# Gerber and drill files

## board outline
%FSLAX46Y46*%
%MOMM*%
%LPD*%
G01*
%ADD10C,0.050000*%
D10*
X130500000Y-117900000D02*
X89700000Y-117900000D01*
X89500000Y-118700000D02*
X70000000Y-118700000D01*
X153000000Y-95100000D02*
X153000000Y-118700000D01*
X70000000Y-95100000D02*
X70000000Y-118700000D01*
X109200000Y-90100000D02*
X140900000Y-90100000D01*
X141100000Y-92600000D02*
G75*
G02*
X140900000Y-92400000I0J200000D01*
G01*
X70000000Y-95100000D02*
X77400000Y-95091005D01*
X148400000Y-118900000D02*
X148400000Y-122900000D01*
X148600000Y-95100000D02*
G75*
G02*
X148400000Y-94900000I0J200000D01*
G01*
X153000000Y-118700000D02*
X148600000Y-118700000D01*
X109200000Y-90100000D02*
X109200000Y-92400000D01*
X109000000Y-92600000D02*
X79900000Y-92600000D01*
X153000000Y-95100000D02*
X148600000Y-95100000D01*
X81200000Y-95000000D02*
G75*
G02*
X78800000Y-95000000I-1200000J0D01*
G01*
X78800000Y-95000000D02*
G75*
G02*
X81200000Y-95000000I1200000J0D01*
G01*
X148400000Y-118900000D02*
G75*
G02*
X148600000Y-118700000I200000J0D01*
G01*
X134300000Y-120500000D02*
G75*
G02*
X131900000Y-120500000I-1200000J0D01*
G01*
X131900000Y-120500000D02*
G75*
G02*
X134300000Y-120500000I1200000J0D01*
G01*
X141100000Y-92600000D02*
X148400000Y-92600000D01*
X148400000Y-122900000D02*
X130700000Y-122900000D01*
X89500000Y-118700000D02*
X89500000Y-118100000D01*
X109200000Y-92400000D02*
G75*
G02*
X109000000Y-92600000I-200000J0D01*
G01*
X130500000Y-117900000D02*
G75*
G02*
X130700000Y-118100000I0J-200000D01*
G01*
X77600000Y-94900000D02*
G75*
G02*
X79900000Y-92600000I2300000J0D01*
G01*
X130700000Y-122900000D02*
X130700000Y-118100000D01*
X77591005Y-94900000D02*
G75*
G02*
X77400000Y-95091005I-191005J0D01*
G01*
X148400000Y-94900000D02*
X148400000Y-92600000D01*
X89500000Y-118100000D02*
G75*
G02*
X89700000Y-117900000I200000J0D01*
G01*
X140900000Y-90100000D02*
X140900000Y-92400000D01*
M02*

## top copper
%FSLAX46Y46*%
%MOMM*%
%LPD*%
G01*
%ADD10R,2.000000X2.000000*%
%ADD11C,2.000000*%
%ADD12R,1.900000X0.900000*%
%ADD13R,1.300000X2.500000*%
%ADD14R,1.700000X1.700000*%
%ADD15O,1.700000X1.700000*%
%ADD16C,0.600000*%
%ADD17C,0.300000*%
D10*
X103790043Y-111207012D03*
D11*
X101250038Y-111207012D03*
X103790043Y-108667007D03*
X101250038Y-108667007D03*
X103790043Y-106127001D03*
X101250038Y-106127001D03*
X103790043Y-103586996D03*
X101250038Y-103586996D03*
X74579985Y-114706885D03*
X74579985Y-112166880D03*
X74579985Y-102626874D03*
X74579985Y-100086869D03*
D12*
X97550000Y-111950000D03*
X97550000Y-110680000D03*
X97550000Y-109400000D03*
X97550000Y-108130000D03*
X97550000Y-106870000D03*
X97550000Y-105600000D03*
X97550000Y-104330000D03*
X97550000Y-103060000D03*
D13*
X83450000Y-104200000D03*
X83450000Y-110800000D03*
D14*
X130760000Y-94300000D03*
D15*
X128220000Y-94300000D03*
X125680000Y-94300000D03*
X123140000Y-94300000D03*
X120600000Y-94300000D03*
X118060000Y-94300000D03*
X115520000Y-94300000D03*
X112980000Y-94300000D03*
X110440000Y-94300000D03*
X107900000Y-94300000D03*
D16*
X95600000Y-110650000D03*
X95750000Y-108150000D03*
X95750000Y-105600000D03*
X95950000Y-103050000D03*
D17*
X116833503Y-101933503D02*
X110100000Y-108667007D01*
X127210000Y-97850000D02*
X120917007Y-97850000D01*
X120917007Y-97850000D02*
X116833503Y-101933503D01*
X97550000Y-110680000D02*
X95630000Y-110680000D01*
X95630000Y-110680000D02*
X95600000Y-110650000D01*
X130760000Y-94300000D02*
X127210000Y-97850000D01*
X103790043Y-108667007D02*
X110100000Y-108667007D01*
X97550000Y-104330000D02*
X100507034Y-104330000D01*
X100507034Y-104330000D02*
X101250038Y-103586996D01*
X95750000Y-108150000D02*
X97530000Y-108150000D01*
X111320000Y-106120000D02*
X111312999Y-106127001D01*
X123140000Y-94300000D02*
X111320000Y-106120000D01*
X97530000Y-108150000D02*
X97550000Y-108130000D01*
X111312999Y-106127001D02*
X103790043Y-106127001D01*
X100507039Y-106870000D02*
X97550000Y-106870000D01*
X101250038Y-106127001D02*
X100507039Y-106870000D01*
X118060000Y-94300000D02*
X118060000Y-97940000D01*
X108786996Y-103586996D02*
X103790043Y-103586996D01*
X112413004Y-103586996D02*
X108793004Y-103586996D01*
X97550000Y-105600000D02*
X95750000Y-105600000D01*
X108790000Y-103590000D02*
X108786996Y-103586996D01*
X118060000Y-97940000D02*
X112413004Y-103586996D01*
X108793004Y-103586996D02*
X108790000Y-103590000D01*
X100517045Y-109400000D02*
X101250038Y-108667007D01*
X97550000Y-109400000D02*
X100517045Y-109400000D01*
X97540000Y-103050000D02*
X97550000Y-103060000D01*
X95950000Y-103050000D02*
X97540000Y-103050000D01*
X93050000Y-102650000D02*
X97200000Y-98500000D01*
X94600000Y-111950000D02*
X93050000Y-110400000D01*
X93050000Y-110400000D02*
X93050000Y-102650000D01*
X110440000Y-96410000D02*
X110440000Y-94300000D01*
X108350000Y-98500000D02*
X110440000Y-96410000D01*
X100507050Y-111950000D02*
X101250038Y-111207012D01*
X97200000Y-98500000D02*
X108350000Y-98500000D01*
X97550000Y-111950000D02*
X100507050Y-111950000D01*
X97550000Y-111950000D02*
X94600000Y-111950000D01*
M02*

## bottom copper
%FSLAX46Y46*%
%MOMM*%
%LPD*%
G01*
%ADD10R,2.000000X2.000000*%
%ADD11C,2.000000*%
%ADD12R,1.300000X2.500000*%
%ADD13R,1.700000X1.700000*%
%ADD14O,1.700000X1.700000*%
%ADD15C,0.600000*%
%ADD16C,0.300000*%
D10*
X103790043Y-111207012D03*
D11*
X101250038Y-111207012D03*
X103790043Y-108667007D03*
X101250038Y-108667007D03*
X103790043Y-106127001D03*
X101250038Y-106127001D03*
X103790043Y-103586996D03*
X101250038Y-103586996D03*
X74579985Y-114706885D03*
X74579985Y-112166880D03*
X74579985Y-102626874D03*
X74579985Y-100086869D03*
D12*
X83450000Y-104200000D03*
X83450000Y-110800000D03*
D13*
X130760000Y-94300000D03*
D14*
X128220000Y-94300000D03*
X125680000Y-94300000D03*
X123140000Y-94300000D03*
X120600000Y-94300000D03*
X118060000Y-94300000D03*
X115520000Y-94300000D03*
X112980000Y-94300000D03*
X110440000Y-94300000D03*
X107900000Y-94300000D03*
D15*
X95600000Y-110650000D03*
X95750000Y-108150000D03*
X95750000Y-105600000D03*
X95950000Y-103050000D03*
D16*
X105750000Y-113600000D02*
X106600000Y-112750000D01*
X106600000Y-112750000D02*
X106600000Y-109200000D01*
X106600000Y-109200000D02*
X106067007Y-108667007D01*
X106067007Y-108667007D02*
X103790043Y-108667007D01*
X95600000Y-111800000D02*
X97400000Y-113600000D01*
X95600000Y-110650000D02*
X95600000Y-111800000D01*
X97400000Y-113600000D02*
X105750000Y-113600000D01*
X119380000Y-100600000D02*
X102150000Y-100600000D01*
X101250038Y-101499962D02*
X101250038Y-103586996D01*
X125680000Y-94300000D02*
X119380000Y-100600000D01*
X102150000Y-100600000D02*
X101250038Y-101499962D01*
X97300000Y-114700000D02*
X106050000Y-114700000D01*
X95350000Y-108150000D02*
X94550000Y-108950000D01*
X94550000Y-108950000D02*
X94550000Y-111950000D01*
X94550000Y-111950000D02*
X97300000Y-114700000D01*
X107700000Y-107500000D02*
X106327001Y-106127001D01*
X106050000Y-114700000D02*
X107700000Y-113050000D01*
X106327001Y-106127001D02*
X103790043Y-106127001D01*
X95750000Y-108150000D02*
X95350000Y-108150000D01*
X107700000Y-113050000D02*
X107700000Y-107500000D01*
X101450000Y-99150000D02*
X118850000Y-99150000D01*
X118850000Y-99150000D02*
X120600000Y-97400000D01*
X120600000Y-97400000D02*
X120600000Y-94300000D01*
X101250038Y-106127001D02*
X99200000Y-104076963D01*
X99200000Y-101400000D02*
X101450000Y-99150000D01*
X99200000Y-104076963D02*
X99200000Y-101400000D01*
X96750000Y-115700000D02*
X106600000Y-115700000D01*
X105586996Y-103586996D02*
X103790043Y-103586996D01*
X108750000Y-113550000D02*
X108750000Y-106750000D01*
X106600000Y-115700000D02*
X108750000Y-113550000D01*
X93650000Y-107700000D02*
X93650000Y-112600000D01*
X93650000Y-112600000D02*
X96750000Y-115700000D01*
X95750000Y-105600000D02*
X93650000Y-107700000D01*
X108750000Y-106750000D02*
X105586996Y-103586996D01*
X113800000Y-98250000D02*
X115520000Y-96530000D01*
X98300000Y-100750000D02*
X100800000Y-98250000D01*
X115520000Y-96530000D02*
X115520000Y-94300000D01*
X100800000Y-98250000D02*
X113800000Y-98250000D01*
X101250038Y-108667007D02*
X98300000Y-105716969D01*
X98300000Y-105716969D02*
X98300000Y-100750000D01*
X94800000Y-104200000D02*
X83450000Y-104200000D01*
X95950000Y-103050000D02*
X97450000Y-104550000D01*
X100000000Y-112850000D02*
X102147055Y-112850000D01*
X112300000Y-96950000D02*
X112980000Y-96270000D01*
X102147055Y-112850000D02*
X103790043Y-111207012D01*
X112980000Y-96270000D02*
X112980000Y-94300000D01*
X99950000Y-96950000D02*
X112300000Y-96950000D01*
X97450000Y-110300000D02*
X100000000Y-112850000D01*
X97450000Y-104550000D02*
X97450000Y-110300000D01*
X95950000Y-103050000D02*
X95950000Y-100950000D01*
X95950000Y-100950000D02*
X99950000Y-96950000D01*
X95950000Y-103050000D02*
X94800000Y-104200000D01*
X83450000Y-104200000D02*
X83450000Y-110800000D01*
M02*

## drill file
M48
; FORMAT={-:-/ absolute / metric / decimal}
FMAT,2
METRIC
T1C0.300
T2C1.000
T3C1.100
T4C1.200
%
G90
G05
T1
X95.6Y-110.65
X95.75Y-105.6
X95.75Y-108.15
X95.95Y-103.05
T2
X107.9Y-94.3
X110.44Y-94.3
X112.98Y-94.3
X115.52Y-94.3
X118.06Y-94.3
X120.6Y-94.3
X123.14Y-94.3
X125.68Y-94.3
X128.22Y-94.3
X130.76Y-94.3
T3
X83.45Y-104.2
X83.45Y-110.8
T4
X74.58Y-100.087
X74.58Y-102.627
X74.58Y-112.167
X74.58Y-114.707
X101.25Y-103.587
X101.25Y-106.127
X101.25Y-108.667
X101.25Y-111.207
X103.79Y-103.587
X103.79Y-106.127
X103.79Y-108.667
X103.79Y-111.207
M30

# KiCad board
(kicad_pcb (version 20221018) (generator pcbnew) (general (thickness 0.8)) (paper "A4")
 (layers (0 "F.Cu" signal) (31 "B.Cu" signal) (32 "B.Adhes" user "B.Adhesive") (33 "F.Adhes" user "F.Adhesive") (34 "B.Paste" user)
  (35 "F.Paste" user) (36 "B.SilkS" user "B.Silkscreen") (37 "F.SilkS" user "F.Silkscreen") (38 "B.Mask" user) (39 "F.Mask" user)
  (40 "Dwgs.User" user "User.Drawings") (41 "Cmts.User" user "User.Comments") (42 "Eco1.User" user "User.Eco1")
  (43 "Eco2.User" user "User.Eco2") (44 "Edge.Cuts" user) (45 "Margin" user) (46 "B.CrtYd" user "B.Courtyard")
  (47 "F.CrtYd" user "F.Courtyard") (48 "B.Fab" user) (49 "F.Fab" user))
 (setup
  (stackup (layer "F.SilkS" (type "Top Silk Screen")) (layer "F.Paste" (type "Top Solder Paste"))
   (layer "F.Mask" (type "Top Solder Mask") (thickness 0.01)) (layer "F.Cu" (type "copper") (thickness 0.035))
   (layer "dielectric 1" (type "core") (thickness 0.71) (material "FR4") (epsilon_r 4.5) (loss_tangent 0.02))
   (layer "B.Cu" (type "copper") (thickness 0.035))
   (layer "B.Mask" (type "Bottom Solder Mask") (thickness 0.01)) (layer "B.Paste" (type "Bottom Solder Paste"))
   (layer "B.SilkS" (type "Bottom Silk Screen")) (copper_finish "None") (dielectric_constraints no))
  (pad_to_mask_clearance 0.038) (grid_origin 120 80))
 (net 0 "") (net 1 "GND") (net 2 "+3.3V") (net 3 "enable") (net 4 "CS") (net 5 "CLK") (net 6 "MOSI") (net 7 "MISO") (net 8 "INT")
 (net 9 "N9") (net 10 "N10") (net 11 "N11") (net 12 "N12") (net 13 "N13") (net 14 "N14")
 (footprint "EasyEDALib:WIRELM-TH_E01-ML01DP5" (layer "F.Cu") (at 89.185014 107.396877)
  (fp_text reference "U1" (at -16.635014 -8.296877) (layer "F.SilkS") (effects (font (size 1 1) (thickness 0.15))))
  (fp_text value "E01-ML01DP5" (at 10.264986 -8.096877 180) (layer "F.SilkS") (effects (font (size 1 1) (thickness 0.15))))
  (pad "1" thru_hole rect (at 14.605029 3.810135 180) (size 2 2) (drill 1.2) (layers "*.Cu" "*.Mask") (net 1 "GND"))
  (pad "2" thru_hole circle (at 12.065024 3.810135) (size 2 2) (drill 1.2) (layers "*.Cu" "*.Mask") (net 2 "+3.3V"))
  (pad "3" thru_hole circle (at 14.605029 1.27013) (size 2 2) (drill 1.2) (layers "*.Cu" "*.Mask") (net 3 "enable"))
  (pad "4" thru_hole circle (at 12.065024 1.27013) (size 2 2) (drill 1.2) (layers "*.Cu" "*.Mask") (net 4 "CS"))
  (pad "5" thru_hole circle (at 14.605029 -1.269876) (size 2 2) (drill 1.2) (layers "*.Cu" "*.Mask") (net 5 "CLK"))
  (pad "6" thru_hole circle (at 12.065024 -1.269876) (size 2 2) (drill 1.2) (layers "*.Cu" "*.Mask") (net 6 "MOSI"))
  (pad "7" thru_hole circle (at 14.605029 -3.809881) (size 2 2) (drill 1.2) (layers "*.Cu" "*.Mask") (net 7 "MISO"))
  (pad "8" thru_hole circle (at 12.065024 -3.809881) (size 2 2) (drill 1.2) (layers "*.Cu" "*.Mask") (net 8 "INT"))
  (pad "9" thru_hole circle (at -14.605029 7.310008) (size 2 2) (drill 1.2) (layers "*.Cu" "*.Mask") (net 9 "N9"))
  (pad "10" thru_hole circle (at -14.605029 4.770003) (size 2 2) (drill 1.2) (layers "*.Cu" "*.Mask") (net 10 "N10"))
  (pad "11" thru_hole circle (at -14.605029 -4.770003) (size 2 2) (drill 1.2) (layers "*.Cu" "*.Mask") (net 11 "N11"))
  (pad "12" thru_hole circle (at -14.605029 -7.310008) (size 2 2) (drill 1.2) (layers "*.Cu" "*.Mask") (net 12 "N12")))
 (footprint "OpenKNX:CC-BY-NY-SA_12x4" (layer "F.Cu") (at 141.325111 119.895111)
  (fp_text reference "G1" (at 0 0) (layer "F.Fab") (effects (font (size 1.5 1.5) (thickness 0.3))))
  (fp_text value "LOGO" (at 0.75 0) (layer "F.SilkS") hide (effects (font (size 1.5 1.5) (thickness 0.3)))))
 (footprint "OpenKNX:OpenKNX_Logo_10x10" (layer "F.Cu") (at 139.42 114.81)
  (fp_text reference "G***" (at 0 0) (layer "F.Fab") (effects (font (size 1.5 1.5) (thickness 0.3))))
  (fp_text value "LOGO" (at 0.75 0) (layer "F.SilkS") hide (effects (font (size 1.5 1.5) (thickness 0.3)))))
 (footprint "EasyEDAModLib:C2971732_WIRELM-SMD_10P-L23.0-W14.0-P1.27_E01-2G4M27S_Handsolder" (layer "F.Cu") (at 90.5 107.5 -90)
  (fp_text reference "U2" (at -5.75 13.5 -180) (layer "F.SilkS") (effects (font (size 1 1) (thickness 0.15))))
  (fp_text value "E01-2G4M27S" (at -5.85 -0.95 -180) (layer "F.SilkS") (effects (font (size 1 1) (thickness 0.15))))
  (pad "1" smd rect (at 4.45 -7.05 180) (size 1.9 0.9) (layers "F.Cu" "F.Paste" "F.Mask") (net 2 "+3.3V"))
  (pad "2" smd rect (at 3.18 -7.05 180) (size 1.9 0.9) (layers "F.Cu" "F.Paste" "F.Mask") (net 3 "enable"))
  (pad "3" smd rect (at 1.9 -7.05 180) (size 1.9 0.9) (layers "F.Cu" "F.Paste" "F.Mask") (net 4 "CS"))
  (pad "4" smd rect (at 0.63 -7.05 180) (size 1.9 0.9) (layers "F.Cu" "F.Paste" "F.Mask") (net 5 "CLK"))
  (pad "5" smd rect (at -0.63 -7.05 180) (size 1.9 0.9) (layers "F.Cu" "F.Paste" "F.Mask") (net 6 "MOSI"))
  (pad "6" smd rect (at -1.9 -7.05 180) (size 1.9 0.9) (layers "F.Cu" "F.Paste" "F.Mask") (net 7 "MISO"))
  (pad "7" smd rect (at -3.17 -7.05 180) (size 1.9 0.9) (layers "F.Cu" "F.Paste" "F.Mask") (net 8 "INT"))
  (pad "8" smd rect (at -4.44 -7.05 180) (size 1.9 0.9) (layers "F.Cu" "F.Paste" "F.Mask") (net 1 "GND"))
  (pad "9" thru_hole rect (at -3.3 7.05 180) (size 1.3 2.5) (drill 1.1) (layers "*.Cu" "*.Mask") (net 1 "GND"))
  (pad "10" thru_hole rect (at 3.3 7.05 180) (size 1.3 2.5) (drill 1.1) (layers "*.Cu" "*.Mask") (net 1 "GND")))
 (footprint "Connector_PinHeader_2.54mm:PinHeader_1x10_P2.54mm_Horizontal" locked (layer "B.Cu") (at 130.76 94.3 90)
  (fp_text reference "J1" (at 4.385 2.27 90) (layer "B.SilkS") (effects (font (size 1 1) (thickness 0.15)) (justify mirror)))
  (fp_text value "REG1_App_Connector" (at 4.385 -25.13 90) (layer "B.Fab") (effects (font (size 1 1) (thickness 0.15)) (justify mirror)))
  (pad "1" thru_hole rect locked (at 0 0 90) (size 1.7 1.7) (drill 1) (layers "*.Cu" "*.Mask") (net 3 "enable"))
  (pad "2" thru_hole oval locked (at 0 -2.54 90) (size 1.7 1.7) (drill 1) (layers "*.Cu" "*.Mask") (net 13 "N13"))
  (pad "3" thru_hole oval locked (at 0 -5.08 90) (size 1.7 1.7) (drill 1) (layers "*.Cu" "*.Mask") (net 8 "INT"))
  (pad "4" thru_hole oval locked (at 0 -7.62 90) (size 1.7 1.7) (drill 1) (layers "*.Cu" "*.Mask") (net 5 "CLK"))
  (pad "5" thru_hole oval locked (at 0 -10.16 90) (size 1.7 1.7) (drill 1) (layers "*.Cu" "*.Mask") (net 6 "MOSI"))
  (pad "6" thru_hole oval locked (at 0 -12.7 90) (size 1.7 1.7) (drill 1) (layers "*.Cu" "*.Mask") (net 7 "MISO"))
  (pad "7" thru_hole oval locked (at 0 -15.24 90) (size 1.7 1.7) (drill 1) (layers "*.Cu" "*.Mask") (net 4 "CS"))
  (pad "8" thru_hole oval locked (at 0 -17.78 90) (size 1.7 1.7) (drill 1) (layers "*.Cu" "*.Mask") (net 1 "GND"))
  (pad "9" thru_hole oval locked (at 0 -20.32 90) (size 1.7 1.7) (drill 1) (layers "*.Cu" "*.Mask") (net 2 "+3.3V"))
  (pad "10" thru_hole oval locked (at 0 -22.86 90) (size 1.7 1.7) (drill 1) (layers "*.Cu" "*.Mask") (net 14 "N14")))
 (gr_line (start 130.5 117.9) (end 89.7 117.9) (stroke (width 0.05) (type solid)) (layer "Edge.Cuts"))
 (gr_line (start 89.5 118.7) (end 70 118.7) (stroke (width 0.05) (type solid)) (layer "Edge.Cuts"))
 (gr_line (start 153 95.1) (end 153 118.7) (stroke (width 0.05) (type solid)) (layer "Edge.Cuts"))
 (gr_line (start 70 95.1) (end 70 118.7) (stroke (width 0.05) (type solid)) (layer "Edge.Cuts"))
 (gr_line (start 109.2 90.1) (end 140.9 90.1) (stroke (width 0.05) (type solid)) (layer "Edge.Cuts"))
 (gr_arc (start 141.1 92.6) (mid 140.958579 92.541421) (end 140.9 92.4) (stroke (width 0.05) (type solid)) (layer "Edge.Cuts"))
 (gr_line (start 70 95.1) (end 77.4 95.091005) (stroke (width 0.05) (type solid)) (layer "Edge.Cuts"))
 (gr_line (start 148.4 118.9) (end 148.4 122.9) (stroke (width 0.05) (type solid)) (layer "Edge.Cuts"))
 (gr_arc (start 148.6 95.1) (mid 148.458579 95.041421) (end 148.4 94.9) (stroke (width 0.05) (type solid)) (layer "Edge.Cuts"))
 (gr_line (start 153 118.7) (end 148.6 118.7) (stroke (width 0.05) (type solid)) (layer "Edge.Cuts"))
 (gr_line (start 109.2 90.1) (end 109.2 92.4) (stroke (width 0.05) (type solid)) (layer "Edge.Cuts"))
 (gr_line (start 109 92.6) (end 79.9 92.6) (stroke (width 0.05) (type solid)) (layer "Edge.Cuts"))
 (gr_line (start 153 95.1) (end 148.6 95.1) (stroke (width 0.05) (type solid)) (layer "Edge.Cuts"))
 (gr_circle (center 80 95) (end 81.2 95) (stroke (width 0.05) (type solid)) (fill none) (layer "Edge.Cuts"))
 (gr_arc (start 148.4 118.9) (mid 148.458579 118.758579) (end 148.6 118.7) (stroke (width 0.05) (type solid)) (layer "Edge.Cuts"))
 (gr_circle (center 133.1 120.5) (end 133.1 121.7) (stroke (width 0.05) (type solid)) (fill none) (layer "Edge.Cuts"))
 (gr_line (start 141.1 92.6) (end 148.4 92.6) (stroke (width 0.05) (type default)) (layer "Edge.Cuts"))
 (gr_line (start 148.4 122.9) (end 130.7 122.9) (stroke (width 0.05) (type solid)) (layer "Edge.Cuts"))
 (gr_line (start 89.5 118.7) (end 89.5 118.1) (stroke (width 0.05) (type default)) (layer "Edge.Cuts"))
 (gr_arc (start 109.2 92.4) (mid 109.141421 92.541421) (end 109 92.6) (stroke (width 0.05) (type default)) (layer "Edge.Cuts"))
 (gr_arc (start 130.5 117.9) (mid 130.641421 117.958579) (end 130.7 118.1) (stroke (width 0.05) (type solid)) (layer "Edge.Cuts"))
 (gr_arc (start 77.6 94.9) (mid 78.273654 93.273654) (end 79.9 92.6) (stroke (width 0.05) (type default)) (layer "Edge.Cuts"))
 (gr_line (start 130.7 122.9) (end 130.7 118.1) (stroke (width 0.05) (type solid)) (layer "Edge.Cuts"))
 (gr_arc (start 77.591005 94.9) (mid 77.535061 95.035061) (end 77.4 95.091005) (stroke (width 0.05) (type default)) (layer "Edge.Cuts"))
 (gr_line (start 148.4 94.9) (end 148.4 92.6) (stroke (width 0.05) (type solid)) (layer "Edge.Cuts"))
 (gr_arc (start 89.5 118.1) (mid 89.558579 117.958579) (end 89.7 117.9) (stroke (width 0.05) (type solid)) (layer "Edge.Cuts"))
 (gr_line (start 140.9 90.1) (end 140.9 92.4) (stroke (width 0.05) (type solid)) (layer "Edge.Cuts"))
 (segment (start 116.833503 101.933503) (end 110.1 108.667007) (width 0.3) (layer "F.Cu") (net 3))
 (segment (start 127.21 97.85) (end 120.917007 97.85) (width 0.3) (layer "F.Cu") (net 3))
 (segment (start 120.917007 97.85) (end 116.833503 101.933503) (width 0.3) (layer "F.Cu") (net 3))
 (segment (start 97.55 110.68) (end 95.63 110.68) (width 0.3) (layer "F.Cu") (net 3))
 (segment (start 95.63 110.68) (end 95.6 110.65) (width 0.3) (layer "F.Cu") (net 3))
 (segment (start 130.76 94.3) (end 127.21 97.85) (width 0.3) (layer "F.Cu") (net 3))
 (segment (start 103.790043 108.667007) (end 110.1 108.667007) (width 0.3) (layer "F.Cu") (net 3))
 (via (at 95.6 110.65) (size 0.6) (drill 0.3) (layers "F.Cu" "B.Cu") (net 3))
 (segment (start 105.75 113.6) (end 106.6 112.75) (width 0.3) (layer "B.Cu") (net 3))
 (segment (start 106.6 112.75) (end 106.6 109.2) (width 0.3) (layer "B.Cu") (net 3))
 (segment (start 106.6 109.2) (end 106.067007 108.667007) (width 0.3) (layer "B.Cu") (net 3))
 (segment (start 106.067007 108.667007) (end 103.790043 108.667007) (width 0.3) (layer "B.Cu") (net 3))
 (segment (start 95.6 111.8) (end 97.4 113.6) (width 0.3) (layer "B.Cu") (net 3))
 (segment (start 95.6 110.65) (end 95.6 111.8) (width 0.3) (layer "B.Cu") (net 3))
 (segment (start 97.4 113.6) (end 105.75 113.6) (width 0.3) (layer "B.Cu") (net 3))
 (segment (start 97.55 104.33) (end 100.507034 104.33) (width 0.3) (layer "F.Cu") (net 8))
 (segment (start 100.507034 104.33) (end 101.250038 103.586996) (width 0.3) (layer "F.Cu") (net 8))
 (segment (start 119.38 100.6) (end 102.15 100.6) (width 0.3) (layer "B.Cu") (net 8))
 (segment (start 101.250038 101.499962) (end 101.250038 103.586996) (width 0.3) (layer "B.Cu") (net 8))
 (segment (start 125.68 94.3) (end 119.38 100.6) (width 0.3) (layer "B.Cu") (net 8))
 (segment (start 102.15 100.6) (end 101.250038 101.499962) (width 0.3) (layer "B.Cu") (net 8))
 (segment (start 95.75 108.15) (end 97.53 108.15) (width 0.3) (layer "F.Cu") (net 5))
 (segment (start 111.32 106.12) (end 111.312999 106.127001) (width 0.3) (layer "F.Cu") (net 5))
 (segment (start 123.14 94.3) (end 111.32 106.12) (width 0.3) (layer "F.Cu") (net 5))
 (segment (start 97.53 108.15) (end 97.55 108.13) (width 0.3) (layer "F.Cu") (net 5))
 (segment (start 111.312999 106.127001) (end 103.790043 106.127001) (width 0.3) (layer "F.Cu") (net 5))
 (via (at 95.75 108.15) (size 0.6) (drill 0.3) (layers "F.Cu" "B.Cu") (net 5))
 (segment (start 97.3 114.7) (end 106.05 114.7) (width 0.3) (layer "B.Cu") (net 5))
 (segment (start 95.35 108.15) (end 94.55 108.95) (width 0.3) (layer "B.Cu") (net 5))
 (segment (start 94.55 108.95) (end 94.55 111.95) (width 0.3) (layer "B.Cu") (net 5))
 (segment (start 94.55 111.95) (end 97.3 114.7) (width 0.3) (layer "B.Cu") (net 5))
 (segment (start 107.7 107.5) (end 106.327001 106.127001) (width 0.3) (layer "B.Cu") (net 5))
 (segment (start 106.05 114.7) (end 107.7 113.05) (width 0.3) (layer "B.Cu") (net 5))
 (segment (start 106.327001 106.127001) (end 103.790043 106.127001) (width 0.3) (layer "B.Cu") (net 5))
 (segment (start 95.75 108.15) (end 95.35 108.15) (width 0.3) (layer "B.Cu") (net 5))
 (segment (start 107.7 113.05) (end 107.7 107.5) (width 0.3) (layer "B.Cu") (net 5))
 (segment (start 100.507039 106.87) (end 97.55 106.87) (width 0.3) (layer "F.Cu") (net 6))
 (segment (start 101.250038 106.127001) (end 100.507039 106.87) (width 0.3) (layer "F.Cu") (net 6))
 (segment (start 101.45 99.15) (end 118.85 99.15) (width 0.3) (layer "B.Cu") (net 6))
 (segment (start 118.85 99.15) (end 120.6 97.4) (width 0.3) (layer "B.Cu") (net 6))
 (segment (start 120.6 97.4) (end 120.6 94.3) (width 0.3) (layer "B.Cu") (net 6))
 (segment (start 101.250038 106.127001) (end 99.2 104.076963) (width 0.3) (layer "B.Cu") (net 6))
 (segment (start 99.2 101.4) (end 101.45 99.15) (width 0.3) (layer "B.Cu") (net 6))
 (segment (start 99.2 104.076963) (end 99.2 101.4) (width 0.3) (layer "B.Cu") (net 6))
 (segment (start 118.06 94.3) (end 118.06 97.94) (width 0.3) (layer "F.Cu") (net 7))
 (segment (start 108.786996 103.586996) (end 103.790043 103.586996) (width 0.3) (layer "F.Cu") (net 7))
 (segment (start 112.413004 103.586996) (end 108.793004 103.586996) (width 0.3) (layer "F.Cu") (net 7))
 (segment (start 97.55 105.6) (end 95.75 105.6) (width 0.3) (layer "F.Cu") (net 7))
 (segment (start 108.79 103.59) (end 108.786996 103.586996) (width 0.3) (layer "F.Cu") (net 7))
 (segment (start 118.06 97.94) (end 112.413004 103.586996) (width 0.3) (layer "F.Cu") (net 7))
 (segment (start 108.793004 103.586996) (end 108.79 103.59) (width 0.3) (layer "F.Cu") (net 7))
 (via (at 95.75 105.6) (size 0.6) (drill 0.3) (layers "F.Cu" "B.Cu") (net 7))
 (segment (start 96.75 115.7) (end 106.6 115.7) (width 0.3) (layer "B.Cu") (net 7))
 (segment (start 105.586996 103.586996) (end 103.790043 103.586996) (width 0.3) (layer "B.Cu") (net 7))
 (segment (start 108.75 113.55) (end 108.75 106.75) (width 0.3) (layer "B.Cu") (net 7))
 (segment (start 106.6 115.7) (end 108.75 113.55) (width 0.3) (layer "B.Cu") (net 7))
 (segment (start 93.65 107.7) (end 93.65 112.6) (width 0.3) (layer "B.Cu") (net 7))
 (segment (start 93.65 112.6) (end 96.75 115.7) (width 0.3) (layer "B.Cu") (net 7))
 (segment (start 95.75 105.6) (end 93.65 107.7) (width 0.3) (layer "B.Cu") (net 7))
 (segment (start 108.75 106.75) (end 105.586996 103.586996) (width 0.3) (layer "B.Cu") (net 7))
 (segment (start 100.517045 109.4) (end 101.250038 108.667007) (width 0.3) (layer "F.Cu") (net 4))
 (segment (start 97.55 109.4) (end 100.517045 109.4) (width 0.3) (layer "F.Cu") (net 4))
 (segment (start 113.8 98.25) (end 115.52 96.53) (width 0.3) (layer "B.Cu") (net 4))
 (segment (start 98.3 100.75) (end 100.8 98.25) (width 0.3) (layer "B.Cu") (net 4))
 (segment (start 115.52 96.53) (end 115.52 94.3) (width 0.3) (layer "B.Cu") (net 4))
 (segment (start 100.8 98.25) (end 113.8 98.25) (width 0.3) (layer "B.Cu") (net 4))
 (segment (start 101.250038 108.667007) (end 98.3 105.716969) (width 0.3) (layer "B.Cu") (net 4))
 (segment (start 98.3 105.716969) (end 98.3 100.75) (width 0.3) (layer "B.Cu") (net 4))
 (segment (start 97.54 103.05) (end 97.55 103.06) (width 0.3) (layer "F.Cu") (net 1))
 (segment (start 95.95 103.05) (end 97.54 103.05) (width 0.3) (layer "F.Cu") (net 1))
 (via (at 95.95 103.05) (size 0.6) (drill 0.3) (layers "F.Cu" "B.Cu") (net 1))
 (segment (start 94.8 104.2) (end 83.45 104.2) (width 0.3) (layer "B.Cu") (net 1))
 (segment (start 95.95 103.05) (end 97.45 104.55) (width 0.3) (layer "B.Cu") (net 1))
 (segment (start 100 112.85) (end 102.147055 112.85) (width 0.3) (layer "B.Cu") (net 1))
 (segment (start 112.3 96.95) (end 112.98 96.27) (width 0.3) (layer "B.Cu") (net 1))
 (segment (start 102.147055 112.85) (end 103.790043 111.207012) (width 0.3) (layer "B.Cu") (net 1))
 (segment (start 112.98 96.27) (end 112.98 94.3) (width 0.3) (layer "B.Cu") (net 1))
 (segment (start 99.95 96.95) (end 112.3 96.95) (width 0.3) (layer "B.Cu") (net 1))
 (segment (start 97.45 110.3) (end 100 112.85) (width 0.3) (layer "B.Cu") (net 1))
 (segment (start 97.45 104.55) (end 97.45 110.3) (width 0.3) (layer "B.Cu") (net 1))
 (segment (start 95.95 103.05) (end 95.95 100.95) (width 0.3) (layer "B.Cu") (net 1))
 (segment (start 95.95 100.95) (end 99.95 96.95) (width 0.3) (layer "B.Cu") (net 1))
 (segment (start 95.95 103.05) (end 94.8 104.2) (width 0.3) (layer "B.Cu") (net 1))
 (segment (start 83.45 104.2) (end 83.45 110.8) (width 0.3) (layer "B.Cu") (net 1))
 (segment (start 93.05 102.65) (end 97.2 98.5) (width 0.3) (layer "F.Cu") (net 2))
 (segment (start 94.6 111.95) (end 93.05 110.4) (width 0.3) (layer "F.Cu") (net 2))
 (segment (start 93.05 110.4) (end 93.05 102.65) (width 0.3) (layer "F.Cu") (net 2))
 (segment (start 110.44 96.41) (end 110.44 94.3) (width 0.3) (layer "F.Cu") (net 2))
 (segment (start 108.35 98.5) (end 110.44 96.41) (width 0.3) (layer "F.Cu") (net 2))
 (segment (start 100.50705 111.95) (end 101.250038 111.207012) (width 0.3) (layer "F.Cu") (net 2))
 (segment (start 97.2 98.5) (end 108.35 98.5) (width 0.3) (layer "F.Cu") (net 2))
 (segment (start 97.55 111.95) (end 100.50705 111.95) (width 0.3) (layer "F.Cu") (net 2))
 (segment (start 97.55 111.95) (end 94.6 111.95) (width 0.3) (layer "F.Cu") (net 2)))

